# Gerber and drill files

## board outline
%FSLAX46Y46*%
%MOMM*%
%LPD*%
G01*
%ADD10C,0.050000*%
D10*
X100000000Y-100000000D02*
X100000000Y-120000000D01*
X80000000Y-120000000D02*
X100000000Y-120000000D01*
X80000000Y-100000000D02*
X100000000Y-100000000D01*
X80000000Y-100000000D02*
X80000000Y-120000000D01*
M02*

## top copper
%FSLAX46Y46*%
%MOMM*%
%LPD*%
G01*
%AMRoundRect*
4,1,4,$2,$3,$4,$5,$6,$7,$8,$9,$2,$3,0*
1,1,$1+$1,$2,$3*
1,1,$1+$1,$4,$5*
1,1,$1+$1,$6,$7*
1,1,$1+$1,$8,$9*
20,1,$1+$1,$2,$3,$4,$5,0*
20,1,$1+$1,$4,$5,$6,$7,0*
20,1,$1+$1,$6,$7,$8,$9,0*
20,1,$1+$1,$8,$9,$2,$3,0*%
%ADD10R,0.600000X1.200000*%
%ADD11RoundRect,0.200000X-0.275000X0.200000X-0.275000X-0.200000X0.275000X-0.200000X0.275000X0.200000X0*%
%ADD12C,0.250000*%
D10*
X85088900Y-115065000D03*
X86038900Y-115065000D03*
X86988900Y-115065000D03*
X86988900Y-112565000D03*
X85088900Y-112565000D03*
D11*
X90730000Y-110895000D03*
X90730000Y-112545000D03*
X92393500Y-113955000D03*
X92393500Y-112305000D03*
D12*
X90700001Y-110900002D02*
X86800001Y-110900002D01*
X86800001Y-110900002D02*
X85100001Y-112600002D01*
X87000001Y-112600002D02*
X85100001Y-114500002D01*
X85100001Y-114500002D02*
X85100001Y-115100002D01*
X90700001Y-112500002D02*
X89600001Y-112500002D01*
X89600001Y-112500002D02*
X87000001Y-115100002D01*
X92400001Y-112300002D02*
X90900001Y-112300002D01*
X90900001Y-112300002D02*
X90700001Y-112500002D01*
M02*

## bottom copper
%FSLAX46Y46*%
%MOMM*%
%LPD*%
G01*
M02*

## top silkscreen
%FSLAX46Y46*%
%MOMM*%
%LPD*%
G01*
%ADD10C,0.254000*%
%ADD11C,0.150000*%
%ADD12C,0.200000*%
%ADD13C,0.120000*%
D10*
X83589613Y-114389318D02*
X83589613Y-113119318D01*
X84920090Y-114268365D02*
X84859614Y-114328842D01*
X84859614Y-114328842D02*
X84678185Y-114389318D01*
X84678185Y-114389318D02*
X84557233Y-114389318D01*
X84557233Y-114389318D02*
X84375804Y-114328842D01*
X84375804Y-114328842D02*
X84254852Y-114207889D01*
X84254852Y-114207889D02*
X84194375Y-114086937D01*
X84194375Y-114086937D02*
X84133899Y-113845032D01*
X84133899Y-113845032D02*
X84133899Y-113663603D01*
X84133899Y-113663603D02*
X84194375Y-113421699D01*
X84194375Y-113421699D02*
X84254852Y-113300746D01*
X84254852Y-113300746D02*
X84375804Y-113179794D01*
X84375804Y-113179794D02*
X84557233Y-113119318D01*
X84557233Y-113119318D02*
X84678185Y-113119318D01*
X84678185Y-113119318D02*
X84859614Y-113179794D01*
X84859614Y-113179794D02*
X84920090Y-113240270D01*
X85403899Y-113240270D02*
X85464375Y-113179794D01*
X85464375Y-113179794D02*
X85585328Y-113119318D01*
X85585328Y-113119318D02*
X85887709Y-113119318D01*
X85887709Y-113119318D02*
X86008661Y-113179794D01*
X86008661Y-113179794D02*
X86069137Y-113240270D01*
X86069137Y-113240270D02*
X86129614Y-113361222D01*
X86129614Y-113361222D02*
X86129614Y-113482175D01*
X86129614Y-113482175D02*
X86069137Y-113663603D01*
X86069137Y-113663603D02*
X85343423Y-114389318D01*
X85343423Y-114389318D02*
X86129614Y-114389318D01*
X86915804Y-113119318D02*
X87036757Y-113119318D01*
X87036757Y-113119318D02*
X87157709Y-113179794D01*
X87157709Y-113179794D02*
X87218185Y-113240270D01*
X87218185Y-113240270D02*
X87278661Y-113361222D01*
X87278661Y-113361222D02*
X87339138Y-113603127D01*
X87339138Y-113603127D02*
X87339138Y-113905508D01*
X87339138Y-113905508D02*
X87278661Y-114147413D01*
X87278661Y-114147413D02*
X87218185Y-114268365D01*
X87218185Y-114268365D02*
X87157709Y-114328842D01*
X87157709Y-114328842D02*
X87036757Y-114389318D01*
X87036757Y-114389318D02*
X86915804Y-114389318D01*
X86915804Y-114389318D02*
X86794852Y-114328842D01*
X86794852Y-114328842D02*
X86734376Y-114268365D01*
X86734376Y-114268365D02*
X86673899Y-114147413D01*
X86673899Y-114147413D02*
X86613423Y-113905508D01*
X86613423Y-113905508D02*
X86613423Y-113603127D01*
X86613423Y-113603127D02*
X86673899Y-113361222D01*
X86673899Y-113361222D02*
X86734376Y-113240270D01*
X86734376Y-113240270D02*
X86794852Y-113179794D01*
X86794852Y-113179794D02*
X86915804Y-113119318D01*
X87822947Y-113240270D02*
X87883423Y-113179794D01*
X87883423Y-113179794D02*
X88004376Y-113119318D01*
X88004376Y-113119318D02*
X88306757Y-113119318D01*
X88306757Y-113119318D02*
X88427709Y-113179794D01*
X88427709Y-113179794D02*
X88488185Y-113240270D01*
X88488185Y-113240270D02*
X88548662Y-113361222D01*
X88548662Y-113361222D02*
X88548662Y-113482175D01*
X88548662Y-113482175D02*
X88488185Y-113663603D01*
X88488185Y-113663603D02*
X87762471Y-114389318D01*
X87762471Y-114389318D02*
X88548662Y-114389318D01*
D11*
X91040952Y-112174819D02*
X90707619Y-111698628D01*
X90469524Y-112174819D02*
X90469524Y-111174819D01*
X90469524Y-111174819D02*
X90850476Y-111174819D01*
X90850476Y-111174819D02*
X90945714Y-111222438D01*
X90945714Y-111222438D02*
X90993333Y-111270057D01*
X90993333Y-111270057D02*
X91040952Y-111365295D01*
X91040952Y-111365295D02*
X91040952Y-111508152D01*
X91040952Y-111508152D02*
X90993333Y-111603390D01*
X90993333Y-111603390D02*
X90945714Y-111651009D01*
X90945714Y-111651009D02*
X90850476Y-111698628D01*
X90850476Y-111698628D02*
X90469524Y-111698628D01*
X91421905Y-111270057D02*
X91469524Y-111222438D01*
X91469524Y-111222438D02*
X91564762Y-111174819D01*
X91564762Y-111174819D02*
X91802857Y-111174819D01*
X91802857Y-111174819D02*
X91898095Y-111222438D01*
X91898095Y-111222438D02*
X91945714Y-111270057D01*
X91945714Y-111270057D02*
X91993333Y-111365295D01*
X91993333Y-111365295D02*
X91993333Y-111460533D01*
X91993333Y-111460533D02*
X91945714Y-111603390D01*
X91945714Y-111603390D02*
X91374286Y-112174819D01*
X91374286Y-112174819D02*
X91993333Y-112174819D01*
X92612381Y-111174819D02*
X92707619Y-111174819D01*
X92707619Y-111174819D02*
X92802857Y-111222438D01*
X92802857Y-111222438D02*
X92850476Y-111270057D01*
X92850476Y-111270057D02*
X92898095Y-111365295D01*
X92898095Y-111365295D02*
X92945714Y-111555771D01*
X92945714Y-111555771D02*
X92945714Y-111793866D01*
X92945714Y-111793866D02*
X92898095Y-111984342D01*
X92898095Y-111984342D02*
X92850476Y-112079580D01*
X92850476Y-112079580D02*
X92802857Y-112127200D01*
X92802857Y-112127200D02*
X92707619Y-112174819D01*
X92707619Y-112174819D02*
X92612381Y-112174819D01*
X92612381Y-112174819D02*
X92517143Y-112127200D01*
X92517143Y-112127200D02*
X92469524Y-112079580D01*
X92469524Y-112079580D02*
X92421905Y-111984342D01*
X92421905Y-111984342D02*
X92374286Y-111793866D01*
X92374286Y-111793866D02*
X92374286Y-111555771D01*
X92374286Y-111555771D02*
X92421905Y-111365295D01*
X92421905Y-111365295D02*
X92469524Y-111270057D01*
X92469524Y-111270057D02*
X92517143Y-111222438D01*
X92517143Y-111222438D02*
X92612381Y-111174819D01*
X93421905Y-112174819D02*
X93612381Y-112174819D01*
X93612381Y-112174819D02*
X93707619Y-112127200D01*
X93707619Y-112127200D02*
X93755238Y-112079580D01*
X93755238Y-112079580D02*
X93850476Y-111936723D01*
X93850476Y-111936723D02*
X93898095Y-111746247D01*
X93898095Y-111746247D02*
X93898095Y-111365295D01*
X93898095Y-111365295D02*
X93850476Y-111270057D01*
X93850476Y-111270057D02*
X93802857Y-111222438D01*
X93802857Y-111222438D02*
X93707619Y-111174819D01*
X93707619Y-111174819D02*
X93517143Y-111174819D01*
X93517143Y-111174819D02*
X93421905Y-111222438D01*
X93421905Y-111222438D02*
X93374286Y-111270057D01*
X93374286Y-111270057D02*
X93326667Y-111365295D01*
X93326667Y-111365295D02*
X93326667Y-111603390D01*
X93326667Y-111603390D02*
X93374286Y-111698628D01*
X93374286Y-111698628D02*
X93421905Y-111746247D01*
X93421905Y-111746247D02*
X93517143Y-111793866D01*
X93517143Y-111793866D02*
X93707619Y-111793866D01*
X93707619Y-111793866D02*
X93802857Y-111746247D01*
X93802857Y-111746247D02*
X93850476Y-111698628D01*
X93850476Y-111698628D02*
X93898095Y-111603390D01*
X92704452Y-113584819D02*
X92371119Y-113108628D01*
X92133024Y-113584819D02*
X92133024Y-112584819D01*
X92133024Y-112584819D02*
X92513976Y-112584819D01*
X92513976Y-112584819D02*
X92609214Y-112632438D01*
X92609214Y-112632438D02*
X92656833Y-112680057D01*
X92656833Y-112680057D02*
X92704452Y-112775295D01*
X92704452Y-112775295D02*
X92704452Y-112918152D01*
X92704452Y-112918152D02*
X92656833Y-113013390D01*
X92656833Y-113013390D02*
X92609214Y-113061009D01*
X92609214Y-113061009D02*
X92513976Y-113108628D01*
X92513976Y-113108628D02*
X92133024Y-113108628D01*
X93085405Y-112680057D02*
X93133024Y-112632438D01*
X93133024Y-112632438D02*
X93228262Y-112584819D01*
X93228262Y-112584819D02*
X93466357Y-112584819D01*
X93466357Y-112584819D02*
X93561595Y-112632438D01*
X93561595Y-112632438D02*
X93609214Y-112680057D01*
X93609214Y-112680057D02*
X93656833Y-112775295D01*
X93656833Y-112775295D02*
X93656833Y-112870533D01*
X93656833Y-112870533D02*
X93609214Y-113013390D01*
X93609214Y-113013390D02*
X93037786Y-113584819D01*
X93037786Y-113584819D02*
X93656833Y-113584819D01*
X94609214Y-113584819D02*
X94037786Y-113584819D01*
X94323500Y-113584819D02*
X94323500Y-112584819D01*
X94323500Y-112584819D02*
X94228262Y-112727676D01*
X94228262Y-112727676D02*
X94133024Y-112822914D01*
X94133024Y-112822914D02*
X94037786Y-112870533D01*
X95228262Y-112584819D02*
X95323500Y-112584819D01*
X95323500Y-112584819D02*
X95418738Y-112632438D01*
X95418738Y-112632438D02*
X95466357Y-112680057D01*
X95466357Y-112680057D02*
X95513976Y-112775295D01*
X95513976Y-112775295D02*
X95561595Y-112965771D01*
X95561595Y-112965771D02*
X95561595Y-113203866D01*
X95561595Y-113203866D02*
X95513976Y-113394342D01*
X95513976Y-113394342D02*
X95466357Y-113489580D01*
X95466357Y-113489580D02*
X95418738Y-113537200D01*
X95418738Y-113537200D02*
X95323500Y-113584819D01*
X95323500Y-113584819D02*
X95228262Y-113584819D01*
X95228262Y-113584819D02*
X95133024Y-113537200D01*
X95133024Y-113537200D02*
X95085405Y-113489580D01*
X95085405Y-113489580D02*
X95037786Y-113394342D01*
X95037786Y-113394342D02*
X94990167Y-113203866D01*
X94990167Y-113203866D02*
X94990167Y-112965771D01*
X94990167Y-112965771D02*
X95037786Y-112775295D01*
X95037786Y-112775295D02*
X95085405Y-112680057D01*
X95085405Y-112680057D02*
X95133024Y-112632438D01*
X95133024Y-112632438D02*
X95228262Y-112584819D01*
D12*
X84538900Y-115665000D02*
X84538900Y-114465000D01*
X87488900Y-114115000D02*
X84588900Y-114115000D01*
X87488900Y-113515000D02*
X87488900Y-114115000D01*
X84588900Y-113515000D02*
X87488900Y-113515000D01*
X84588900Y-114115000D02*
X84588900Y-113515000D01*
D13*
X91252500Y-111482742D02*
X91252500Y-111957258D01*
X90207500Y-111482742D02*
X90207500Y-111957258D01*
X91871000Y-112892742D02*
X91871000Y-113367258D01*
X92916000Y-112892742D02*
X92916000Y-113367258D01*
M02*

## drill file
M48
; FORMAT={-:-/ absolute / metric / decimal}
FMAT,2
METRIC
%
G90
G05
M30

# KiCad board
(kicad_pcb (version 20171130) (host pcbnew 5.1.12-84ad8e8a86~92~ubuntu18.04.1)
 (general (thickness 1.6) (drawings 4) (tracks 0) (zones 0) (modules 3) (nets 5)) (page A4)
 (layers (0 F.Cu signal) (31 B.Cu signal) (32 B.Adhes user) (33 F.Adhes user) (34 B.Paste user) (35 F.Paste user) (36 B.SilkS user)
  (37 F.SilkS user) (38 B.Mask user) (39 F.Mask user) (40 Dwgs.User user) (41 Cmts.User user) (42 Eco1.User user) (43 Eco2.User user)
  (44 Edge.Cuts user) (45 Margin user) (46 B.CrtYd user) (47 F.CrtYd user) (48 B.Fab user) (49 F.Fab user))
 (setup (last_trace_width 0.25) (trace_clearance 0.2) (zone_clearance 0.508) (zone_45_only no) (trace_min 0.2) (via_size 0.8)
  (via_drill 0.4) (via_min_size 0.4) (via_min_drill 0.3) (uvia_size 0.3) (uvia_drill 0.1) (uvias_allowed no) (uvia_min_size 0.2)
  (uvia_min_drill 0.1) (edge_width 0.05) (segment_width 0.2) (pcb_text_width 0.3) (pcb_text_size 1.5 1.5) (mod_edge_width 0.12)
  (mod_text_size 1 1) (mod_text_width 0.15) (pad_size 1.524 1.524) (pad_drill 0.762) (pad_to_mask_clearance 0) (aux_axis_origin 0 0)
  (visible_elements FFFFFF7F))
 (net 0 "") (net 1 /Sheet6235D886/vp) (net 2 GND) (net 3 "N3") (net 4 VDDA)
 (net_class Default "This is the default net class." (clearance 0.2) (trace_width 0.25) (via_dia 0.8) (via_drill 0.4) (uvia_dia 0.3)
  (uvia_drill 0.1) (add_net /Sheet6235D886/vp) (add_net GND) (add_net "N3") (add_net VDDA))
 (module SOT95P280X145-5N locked (layer F.Cu) (at 86.038900 113.815000 90.000000)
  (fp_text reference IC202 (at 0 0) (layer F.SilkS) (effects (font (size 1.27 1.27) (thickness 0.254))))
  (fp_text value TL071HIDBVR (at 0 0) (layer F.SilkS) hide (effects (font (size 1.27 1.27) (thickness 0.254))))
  (fp_line (start -1.85 -1.5) (end -0.65 -1.5) (layer F.SilkS) (width 0.2))
  (fp_line (start -0.3 1.45) (end -0.3 -1.45) (layer F.SilkS) (width 0.2))
  (fp_line (start 0.3 1.45) (end -0.3 1.45) (layer F.SilkS) (width 0.2))
  (fp_line (start 0.3 -1.45) (end 0.3 1.45) (layer F.SilkS) (width 0.2))
  (fp_line (start -0.3 -1.45) (end 0.3 -1.45) (layer F.SilkS) (width 0.2))
  (pad 1 smd rect (at -1.25 -0.95 180.000000) (size 0.6 1.2) (layers F.Cu F.Mask F.Paste) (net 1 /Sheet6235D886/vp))
  (pad 2 smd rect (at -1.25 0 180.000000) (size 0.6 1.2) (layers F.Cu F.Mask F.Paste) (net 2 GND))
  (pad 3 smd rect (at -1.25 0.95 180.000000) (size 0.6 1.2) (layers F.Cu F.Mask F.Paste) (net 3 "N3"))
  (pad 4 smd rect (at 1.25 0.95 180.000000) (size 0.6 1.2) (layers F.Cu F.Mask F.Paste) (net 1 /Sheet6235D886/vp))
  (pad 5 smd rect (at 1.25 -0.95 180.000000) (size 0.6 1.2) (layers F.Cu F.Mask F.Paste) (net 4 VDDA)))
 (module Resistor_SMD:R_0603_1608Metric (layer F.Cu) (at 90.730000 111.720000 270.000000)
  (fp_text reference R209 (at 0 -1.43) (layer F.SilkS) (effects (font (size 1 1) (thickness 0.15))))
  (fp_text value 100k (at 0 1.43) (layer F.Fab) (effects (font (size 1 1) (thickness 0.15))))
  (fp_line (start -0.237258 -0.5225) (end 0.237258 -0.5225) (layer F.SilkS) (width 0.12))
  (fp_line (start -0.237258 0.5225) (end 0.237258 0.5225) (layer F.SilkS) (width 0.12))
  (pad 1 smd roundrect (at -0.825 0 270.000000) (size 0.8 0.95) (layers F.Cu F.Mask F.Paste) (roundrect_rratio 0.25) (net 4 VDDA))
  (pad 2 smd roundrect (at 0.825 0 270.000000) (size 0.8 0.95) (layers F.Cu F.Mask F.Paste) (roundrect_rratio 0.25) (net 3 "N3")))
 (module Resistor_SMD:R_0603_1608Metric (layer F.Cu) (at 92.393500 113.130000 270.000000)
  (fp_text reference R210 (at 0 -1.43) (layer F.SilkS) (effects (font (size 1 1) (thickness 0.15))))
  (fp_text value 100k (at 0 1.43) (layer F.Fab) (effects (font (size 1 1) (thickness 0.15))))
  (fp_line (start -0.237258 0.5225) (end 0.237258 0.5225) (layer F.SilkS) (width 0.12))
  (fp_line (start -0.237258 -0.5225) (end 0.237258 -0.5225) (layer F.SilkS) (width 0.12))
  (pad 2 smd roundrect (at 0.825 0 270.000000) (size 0.8 0.95) (layers F.Cu F.Mask F.Paste) (roundrect_rratio 0.25) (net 2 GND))
  (pad 1 smd roundrect (at -0.825 0 270.000000) (size 0.8 0.95) (layers F.Cu F.Mask F.Paste) (roundrect_rratio 0.25) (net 3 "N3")))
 (gr_line (start 100 100) (end 100 120) (layer Edge.Cuts) (width 0.05))
 (gr_line (start 80 120) (end 100 120) (layer Edge.Cuts) (width 0.05))
 (gr_line (start 80 100) (end 100 100) (layer Edge.Cuts) (width 0.05))
 (gr_line (start 80 100) (end 80 120) (layer Edge.Cuts) (width 0.05))
 (segment (start 90.700001 110.900002) (end 86.800001 110.900002) (width 0.250000) (layer F.Cu) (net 4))
 (segment (start 86.800001 110.900002) (end 85.100001 112.600002) (width 0.250000) (layer F.Cu) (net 4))
 (segment (start 87.000001 112.600002) (end 85.100001 114.500002) (width 0.250000) (layer F.Cu) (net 1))
 (segment (start 85.100001 114.500002) (end 85.100001 115.100002) (width 0.250000) (layer F.Cu) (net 1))
 (segment (start 90.700001 112.500002) (end 89.600001 112.500002) (width 0.250000) (layer F.Cu) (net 3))
 (segment (start 89.600001 112.500002) (end 87.000001 115.100002) (width 0.250000) (layer F.Cu) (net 3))
 (segment (start 92.400001 112.300002) (end 90.900001 112.300002) (width 0.250000) (layer F.Cu) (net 3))
 (segment (start 90.900001 112.300002) (end 90.700001 112.500002) (width 0.250000) (layer F.Cu) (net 3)))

